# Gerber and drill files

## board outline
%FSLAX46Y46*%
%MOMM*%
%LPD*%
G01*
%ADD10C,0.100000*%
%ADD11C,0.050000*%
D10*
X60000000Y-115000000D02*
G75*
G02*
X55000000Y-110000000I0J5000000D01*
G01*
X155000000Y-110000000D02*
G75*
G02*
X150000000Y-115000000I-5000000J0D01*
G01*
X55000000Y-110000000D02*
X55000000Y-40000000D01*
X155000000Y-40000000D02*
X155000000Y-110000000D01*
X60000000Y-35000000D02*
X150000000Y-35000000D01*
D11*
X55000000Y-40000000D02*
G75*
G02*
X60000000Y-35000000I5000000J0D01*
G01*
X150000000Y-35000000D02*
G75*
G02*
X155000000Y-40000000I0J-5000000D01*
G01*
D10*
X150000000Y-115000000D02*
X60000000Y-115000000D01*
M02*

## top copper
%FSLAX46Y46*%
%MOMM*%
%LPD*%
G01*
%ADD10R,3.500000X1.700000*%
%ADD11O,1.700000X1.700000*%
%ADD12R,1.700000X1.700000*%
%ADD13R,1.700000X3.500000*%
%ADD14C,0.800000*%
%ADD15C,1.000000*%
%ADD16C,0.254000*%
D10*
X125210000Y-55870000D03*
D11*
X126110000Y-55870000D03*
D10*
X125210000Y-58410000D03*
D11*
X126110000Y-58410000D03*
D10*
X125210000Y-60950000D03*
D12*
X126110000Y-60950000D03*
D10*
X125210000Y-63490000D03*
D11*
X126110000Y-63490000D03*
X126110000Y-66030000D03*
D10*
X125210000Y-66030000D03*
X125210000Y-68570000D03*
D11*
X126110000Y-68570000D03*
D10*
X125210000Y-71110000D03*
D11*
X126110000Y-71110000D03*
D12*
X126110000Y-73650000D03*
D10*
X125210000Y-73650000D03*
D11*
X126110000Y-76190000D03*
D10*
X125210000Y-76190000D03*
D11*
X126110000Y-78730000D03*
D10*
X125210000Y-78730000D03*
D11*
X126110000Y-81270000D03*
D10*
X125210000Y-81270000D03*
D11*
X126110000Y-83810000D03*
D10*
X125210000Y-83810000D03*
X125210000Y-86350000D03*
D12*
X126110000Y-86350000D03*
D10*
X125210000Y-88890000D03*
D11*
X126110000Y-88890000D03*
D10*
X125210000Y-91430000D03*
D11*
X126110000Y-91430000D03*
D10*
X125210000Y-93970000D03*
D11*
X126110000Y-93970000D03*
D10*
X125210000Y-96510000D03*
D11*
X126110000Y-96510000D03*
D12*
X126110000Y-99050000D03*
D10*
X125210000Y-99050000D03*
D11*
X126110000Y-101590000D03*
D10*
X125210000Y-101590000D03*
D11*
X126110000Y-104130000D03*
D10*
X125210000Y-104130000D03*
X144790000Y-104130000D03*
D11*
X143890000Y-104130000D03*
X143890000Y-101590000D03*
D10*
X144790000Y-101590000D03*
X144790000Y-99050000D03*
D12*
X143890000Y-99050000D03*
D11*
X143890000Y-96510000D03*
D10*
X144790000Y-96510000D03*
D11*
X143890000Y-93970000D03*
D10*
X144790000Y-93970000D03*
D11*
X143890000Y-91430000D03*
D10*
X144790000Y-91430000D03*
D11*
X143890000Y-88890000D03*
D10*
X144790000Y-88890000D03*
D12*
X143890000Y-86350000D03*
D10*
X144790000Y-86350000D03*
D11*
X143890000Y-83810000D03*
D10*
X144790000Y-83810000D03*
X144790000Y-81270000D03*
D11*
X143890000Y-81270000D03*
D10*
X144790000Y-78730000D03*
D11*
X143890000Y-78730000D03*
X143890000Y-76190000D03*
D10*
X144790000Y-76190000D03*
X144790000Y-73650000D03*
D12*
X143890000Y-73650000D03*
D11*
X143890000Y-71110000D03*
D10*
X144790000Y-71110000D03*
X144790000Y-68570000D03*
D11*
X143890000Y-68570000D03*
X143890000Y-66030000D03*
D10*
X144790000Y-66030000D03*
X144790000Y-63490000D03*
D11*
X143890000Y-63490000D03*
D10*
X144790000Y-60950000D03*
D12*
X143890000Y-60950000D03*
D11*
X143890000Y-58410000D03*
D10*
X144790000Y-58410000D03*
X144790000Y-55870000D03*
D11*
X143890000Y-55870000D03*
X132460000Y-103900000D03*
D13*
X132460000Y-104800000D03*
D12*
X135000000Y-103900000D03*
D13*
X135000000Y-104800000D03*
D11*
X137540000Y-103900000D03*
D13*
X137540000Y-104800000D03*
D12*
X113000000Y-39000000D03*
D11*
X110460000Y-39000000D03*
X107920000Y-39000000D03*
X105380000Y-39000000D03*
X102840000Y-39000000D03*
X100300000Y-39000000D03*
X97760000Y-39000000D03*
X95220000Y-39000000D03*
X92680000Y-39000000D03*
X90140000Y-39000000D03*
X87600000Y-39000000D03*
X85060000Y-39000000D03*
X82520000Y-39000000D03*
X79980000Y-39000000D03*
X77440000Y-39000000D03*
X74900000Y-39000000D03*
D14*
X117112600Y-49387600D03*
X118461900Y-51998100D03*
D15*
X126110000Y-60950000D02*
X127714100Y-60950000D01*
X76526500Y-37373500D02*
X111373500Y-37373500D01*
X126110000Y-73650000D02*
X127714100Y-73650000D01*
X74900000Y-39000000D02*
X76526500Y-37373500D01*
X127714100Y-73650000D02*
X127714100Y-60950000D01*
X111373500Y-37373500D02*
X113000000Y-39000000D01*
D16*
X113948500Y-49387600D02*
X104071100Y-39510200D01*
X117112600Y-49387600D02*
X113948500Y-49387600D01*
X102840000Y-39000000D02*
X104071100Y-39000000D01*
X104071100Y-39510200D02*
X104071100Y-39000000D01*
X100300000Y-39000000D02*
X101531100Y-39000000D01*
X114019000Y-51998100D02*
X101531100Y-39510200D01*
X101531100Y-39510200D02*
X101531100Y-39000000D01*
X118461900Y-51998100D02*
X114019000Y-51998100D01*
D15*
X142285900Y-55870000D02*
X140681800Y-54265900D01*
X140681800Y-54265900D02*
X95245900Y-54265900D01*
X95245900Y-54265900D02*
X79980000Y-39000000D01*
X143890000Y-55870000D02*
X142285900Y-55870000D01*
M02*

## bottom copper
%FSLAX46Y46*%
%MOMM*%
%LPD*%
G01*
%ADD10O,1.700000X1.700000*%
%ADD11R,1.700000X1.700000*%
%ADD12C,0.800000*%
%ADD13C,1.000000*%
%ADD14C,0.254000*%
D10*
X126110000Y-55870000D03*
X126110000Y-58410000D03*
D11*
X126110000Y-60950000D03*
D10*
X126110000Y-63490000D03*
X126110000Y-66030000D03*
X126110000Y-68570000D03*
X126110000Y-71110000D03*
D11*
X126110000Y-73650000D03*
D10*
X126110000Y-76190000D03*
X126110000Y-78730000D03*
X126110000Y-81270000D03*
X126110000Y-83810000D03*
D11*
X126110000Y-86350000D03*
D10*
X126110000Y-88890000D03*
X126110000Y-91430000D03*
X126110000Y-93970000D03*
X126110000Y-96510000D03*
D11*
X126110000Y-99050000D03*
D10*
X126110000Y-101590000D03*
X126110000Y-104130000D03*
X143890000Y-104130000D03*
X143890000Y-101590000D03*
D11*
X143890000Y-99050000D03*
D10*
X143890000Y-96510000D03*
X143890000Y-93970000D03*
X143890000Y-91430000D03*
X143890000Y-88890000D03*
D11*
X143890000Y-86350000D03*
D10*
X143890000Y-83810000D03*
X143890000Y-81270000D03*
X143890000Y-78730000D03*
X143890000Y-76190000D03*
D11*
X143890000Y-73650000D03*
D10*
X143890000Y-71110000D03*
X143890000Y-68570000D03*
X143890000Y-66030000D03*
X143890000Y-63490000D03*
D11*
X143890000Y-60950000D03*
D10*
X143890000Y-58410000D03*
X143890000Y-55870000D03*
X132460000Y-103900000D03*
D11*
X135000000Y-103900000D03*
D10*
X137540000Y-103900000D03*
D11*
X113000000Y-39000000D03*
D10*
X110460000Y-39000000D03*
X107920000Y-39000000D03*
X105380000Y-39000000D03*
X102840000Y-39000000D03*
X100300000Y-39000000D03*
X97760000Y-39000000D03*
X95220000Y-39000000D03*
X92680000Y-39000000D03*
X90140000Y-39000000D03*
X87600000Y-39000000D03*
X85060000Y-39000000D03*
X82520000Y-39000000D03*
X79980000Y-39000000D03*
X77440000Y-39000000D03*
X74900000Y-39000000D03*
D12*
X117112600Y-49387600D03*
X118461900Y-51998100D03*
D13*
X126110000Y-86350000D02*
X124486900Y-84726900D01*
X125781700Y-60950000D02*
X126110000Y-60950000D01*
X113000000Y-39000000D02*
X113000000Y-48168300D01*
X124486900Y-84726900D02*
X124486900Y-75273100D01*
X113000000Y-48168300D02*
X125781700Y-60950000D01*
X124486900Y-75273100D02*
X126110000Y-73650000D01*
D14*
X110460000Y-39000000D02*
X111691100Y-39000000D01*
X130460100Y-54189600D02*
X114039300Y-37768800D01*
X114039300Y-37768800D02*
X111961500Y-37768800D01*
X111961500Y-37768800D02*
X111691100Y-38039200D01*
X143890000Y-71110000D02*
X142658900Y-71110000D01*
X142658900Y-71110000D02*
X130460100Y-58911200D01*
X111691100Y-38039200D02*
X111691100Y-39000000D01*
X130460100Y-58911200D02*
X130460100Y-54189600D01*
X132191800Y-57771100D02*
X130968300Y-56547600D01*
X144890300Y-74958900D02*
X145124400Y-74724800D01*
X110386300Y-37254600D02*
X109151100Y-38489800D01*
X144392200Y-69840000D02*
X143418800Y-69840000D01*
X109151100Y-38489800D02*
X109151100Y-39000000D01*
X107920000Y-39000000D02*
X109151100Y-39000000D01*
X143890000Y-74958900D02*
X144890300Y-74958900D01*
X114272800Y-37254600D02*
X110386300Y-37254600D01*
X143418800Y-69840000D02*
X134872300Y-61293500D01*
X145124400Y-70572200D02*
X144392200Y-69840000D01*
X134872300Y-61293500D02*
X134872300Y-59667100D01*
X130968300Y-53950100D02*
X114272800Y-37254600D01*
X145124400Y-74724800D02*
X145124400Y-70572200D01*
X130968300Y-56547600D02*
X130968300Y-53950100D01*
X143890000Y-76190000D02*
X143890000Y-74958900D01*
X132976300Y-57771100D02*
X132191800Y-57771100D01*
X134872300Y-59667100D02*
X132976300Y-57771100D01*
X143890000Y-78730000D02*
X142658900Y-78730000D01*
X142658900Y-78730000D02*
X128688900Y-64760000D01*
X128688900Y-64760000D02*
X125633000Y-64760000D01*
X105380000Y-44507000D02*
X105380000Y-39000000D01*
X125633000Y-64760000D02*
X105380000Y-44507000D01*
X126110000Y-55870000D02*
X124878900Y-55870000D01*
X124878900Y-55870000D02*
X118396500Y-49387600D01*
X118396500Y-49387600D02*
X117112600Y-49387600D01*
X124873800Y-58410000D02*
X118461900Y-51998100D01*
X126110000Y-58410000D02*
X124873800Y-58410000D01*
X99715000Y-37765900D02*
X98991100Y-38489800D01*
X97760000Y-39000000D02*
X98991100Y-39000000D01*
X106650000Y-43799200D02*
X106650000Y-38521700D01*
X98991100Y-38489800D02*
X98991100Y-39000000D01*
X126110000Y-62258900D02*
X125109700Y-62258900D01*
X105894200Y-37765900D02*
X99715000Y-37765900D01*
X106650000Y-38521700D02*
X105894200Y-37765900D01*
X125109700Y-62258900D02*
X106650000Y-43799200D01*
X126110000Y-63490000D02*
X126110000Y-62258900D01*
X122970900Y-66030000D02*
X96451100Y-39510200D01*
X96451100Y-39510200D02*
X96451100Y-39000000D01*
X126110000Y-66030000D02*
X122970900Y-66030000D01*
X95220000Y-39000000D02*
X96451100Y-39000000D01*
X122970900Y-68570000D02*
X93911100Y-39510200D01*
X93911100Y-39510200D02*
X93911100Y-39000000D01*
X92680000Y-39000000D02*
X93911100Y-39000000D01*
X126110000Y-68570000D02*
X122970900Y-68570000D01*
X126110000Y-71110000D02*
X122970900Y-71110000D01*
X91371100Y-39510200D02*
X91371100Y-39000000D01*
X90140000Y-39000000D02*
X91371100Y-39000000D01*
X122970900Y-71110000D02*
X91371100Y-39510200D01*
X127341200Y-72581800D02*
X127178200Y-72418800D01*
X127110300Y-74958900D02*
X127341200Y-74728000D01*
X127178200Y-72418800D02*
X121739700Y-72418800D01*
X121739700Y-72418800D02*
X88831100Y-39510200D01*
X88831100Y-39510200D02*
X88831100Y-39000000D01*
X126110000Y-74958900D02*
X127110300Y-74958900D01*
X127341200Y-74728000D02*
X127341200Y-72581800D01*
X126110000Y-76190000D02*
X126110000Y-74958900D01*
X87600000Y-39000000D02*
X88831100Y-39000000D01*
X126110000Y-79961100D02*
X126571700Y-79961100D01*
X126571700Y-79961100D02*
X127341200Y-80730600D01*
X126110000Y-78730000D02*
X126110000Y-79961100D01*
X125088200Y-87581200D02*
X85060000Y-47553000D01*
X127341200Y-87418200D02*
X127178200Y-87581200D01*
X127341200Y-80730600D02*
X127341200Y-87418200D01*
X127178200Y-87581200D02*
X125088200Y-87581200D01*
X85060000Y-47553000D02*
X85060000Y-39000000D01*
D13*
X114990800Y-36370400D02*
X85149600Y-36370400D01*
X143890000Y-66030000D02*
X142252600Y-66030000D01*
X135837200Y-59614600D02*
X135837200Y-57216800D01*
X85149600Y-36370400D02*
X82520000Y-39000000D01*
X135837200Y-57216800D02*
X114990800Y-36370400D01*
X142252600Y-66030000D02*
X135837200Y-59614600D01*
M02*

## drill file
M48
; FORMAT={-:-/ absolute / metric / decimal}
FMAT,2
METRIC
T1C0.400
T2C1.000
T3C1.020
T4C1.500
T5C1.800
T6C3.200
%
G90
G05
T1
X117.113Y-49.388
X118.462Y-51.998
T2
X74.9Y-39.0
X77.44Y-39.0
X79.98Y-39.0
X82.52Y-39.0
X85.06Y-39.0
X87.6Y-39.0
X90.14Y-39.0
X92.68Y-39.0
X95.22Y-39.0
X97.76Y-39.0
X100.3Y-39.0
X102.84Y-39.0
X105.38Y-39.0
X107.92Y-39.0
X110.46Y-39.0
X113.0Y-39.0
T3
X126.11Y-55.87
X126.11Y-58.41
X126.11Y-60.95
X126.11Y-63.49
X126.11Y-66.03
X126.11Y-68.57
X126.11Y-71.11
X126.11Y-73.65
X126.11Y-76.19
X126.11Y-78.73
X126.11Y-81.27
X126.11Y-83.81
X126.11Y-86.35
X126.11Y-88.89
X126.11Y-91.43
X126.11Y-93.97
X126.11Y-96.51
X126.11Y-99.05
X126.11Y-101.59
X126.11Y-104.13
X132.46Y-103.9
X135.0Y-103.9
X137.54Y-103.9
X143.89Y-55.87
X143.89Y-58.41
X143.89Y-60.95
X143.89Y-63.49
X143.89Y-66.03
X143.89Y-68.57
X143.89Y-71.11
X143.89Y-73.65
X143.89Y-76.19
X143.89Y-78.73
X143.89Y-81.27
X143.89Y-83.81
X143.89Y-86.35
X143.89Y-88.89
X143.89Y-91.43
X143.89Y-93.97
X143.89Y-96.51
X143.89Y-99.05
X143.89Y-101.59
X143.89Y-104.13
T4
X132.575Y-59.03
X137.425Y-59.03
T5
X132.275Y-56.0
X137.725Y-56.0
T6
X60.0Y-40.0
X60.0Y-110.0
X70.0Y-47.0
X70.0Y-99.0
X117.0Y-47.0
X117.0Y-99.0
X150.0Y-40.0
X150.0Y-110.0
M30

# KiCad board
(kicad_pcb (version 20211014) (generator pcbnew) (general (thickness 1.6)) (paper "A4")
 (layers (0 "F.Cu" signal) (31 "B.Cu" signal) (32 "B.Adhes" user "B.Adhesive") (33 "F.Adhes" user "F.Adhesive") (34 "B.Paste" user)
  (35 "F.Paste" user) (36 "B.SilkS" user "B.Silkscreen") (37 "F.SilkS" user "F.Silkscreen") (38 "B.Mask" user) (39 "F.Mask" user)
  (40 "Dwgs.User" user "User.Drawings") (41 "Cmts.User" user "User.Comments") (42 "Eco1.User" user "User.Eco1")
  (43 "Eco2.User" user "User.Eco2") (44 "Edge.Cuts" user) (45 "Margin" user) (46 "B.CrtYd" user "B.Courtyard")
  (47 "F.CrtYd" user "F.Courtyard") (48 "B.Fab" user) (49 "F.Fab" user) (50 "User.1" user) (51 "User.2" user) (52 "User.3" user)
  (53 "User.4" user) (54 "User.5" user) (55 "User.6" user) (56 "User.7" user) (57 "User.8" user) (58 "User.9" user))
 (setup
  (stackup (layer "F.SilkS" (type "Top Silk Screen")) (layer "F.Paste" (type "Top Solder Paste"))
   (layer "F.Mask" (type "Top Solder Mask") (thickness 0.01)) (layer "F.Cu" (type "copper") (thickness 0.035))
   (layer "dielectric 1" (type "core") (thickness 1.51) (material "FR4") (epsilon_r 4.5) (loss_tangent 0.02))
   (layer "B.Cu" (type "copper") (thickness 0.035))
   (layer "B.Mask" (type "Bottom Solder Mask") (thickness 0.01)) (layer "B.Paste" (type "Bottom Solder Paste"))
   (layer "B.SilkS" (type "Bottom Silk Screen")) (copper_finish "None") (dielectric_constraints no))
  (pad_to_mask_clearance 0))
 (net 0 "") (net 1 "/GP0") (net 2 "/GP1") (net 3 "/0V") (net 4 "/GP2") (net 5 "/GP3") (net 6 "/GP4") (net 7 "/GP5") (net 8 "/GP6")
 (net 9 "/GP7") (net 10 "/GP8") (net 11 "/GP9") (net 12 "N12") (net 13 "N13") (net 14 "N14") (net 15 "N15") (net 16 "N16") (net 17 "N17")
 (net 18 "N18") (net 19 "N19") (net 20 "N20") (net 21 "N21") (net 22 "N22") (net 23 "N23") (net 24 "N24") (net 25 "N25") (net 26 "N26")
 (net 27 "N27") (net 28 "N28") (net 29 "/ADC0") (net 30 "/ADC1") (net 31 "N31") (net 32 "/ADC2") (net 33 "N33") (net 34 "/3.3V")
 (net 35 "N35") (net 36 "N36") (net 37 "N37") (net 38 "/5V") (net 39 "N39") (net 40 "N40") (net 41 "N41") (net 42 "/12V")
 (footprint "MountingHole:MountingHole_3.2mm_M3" (layer "F.Cu") (at 117 99)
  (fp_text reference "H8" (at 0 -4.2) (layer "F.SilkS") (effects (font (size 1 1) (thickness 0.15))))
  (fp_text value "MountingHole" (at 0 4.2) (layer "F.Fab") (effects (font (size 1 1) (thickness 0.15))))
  (pad "" np_thru_hole circle (at 0 0) (size 3.2 3.2) (drill 3.2) (layers *.Cu *.Mask)))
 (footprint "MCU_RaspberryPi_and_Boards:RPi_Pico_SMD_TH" (layer "F.Cu") (at 135 80)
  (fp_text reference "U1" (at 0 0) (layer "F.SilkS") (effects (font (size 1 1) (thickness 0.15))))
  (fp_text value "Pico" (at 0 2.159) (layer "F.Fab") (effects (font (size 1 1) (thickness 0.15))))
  (pad "" np_thru_hole oval (at -2.725 -24) (size 1.8 1.8) (drill 1.8) (layers *.Cu *.Mask))
  (pad "" np_thru_hole oval (at -2.425 -20.97) (size 1.5 1.5) (drill 1.5) (layers *.Cu *.Mask))
  (pad "" np_thru_hole oval (at 2.425 -20.97) (size 1.5 1.5) (drill 1.5) (layers *.Cu *.Mask))
  (pad "" np_thru_hole oval (at 2.725 -24) (size 1.8 1.8) (drill 1.8) (layers *.Cu *.Mask))
  (pad "1" smd rect (at -8.89 -24.13) (size 3.5 1.7) (drill (offset -0.9 0)) (layers "F.Cu" "F.Mask") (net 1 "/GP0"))
  (pad "1" thru_hole oval (at -8.89 -24.13) (size 1.7 1.7) (drill 1.02) (layers *.Cu *.Mask) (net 1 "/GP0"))
  (pad "2" smd rect (at -8.89 -21.59) (size 3.5 1.7) (drill (offset -0.9 0)) (layers "F.Cu" "F.Mask") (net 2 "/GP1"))
  (pad "2" thru_hole oval (at -8.89 -21.59) (size 1.7 1.7) (drill 1.02) (layers *.Cu *.Mask) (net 2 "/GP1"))
  (pad "3" smd rect (at -8.89 -19.05) (size 3.5 1.7) (drill (offset -0.9 0)) (layers "F.Cu" "F.Mask") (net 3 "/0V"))
  (pad "3" thru_hole rect (at -8.89 -19.05) (size 1.7 1.7) (drill 1.02) (layers *.Cu *.Mask) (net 3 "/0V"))
  (pad "4" smd rect (at -8.89 -16.51) (size 3.5 1.7) (drill (offset -0.9 0)) (layers "F.Cu" "F.Mask") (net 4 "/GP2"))
  (pad "4" thru_hole oval (at -8.89 -16.51) (size 1.7 1.7) (drill 1.02) (layers *.Cu *.Mask) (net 4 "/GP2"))
  (pad "5" thru_hole oval (at -8.89 -13.97) (size 1.7 1.7) (drill 1.02) (layers *.Cu *.Mask) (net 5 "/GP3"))
  (pad "5" smd rect (at -8.89 -13.97) (size 3.5 1.7) (drill (offset -0.9 0)) (layers "F.Cu" "F.Mask") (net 5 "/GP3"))
  (pad "6" smd rect (at -8.89 -11.43) (size 3.5 1.7) (drill (offset -0.9 0)) (layers "F.Cu" "F.Mask") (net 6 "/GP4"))
  (pad "6" thru_hole oval (at -8.89 -11.43) (size 1.7 1.7) (drill 1.02) (layers *.Cu *.Mask) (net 6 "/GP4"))
  (pad "7" smd rect (at -8.89 -8.89) (size 3.5 1.7) (drill (offset -0.9 0)) (layers "F.Cu" "F.Mask") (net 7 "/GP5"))
  (pad "7" thru_hole oval (at -8.89 -8.89) (size 1.7 1.7) (drill 1.02) (layers *.Cu *.Mask) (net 7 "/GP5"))
  (pad "8" thru_hole rect (at -8.89 -6.35) (size 1.7 1.7) (drill 1.02) (layers *.Cu *.Mask) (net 3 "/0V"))
  (pad "8" smd rect (at -8.89 -6.35) (size 3.5 1.7) (drill (offset -0.9 0)) (layers "F.Cu" "F.Mask") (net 3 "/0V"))
  (pad "9" thru_hole oval (at -8.89 -3.81) (size 1.7 1.7) (drill 1.02) (layers *.Cu *.Mask) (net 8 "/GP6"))
  (pad "9" smd rect (at -8.89 -3.81) (size 3.5 1.7) (drill (offset -0.9 0)) (layers "F.Cu" "F.Mask") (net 8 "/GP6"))
  (pad "10" thru_hole oval (at -8.89 -1.27) (size 1.7 1.7) (drill 1.02) (layers *.Cu *.Mask) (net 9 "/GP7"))
  (pad "10" smd rect (at -8.89 -1.27) (size 3.5 1.7) (drill (offset -0.9 0)) (layers "F.Cu" "F.Mask") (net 9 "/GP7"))
  (pad "11" thru_hole oval (at -8.89 1.27) (size 1.7 1.7) (drill 1.02) (layers *.Cu *.Mask) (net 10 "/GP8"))
  (pad "11" smd rect (at -8.89 1.27) (size 3.5 1.7) (drill (offset -0.9 0)) (layers "F.Cu" "F.Mask") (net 10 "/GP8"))
  (pad "12" thru_hole oval (at -8.89 3.81) (size 1.7 1.7) (drill 1.02) (layers *.Cu *.Mask) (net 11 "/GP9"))
  (pad "12" smd rect (at -8.89 3.81) (size 3.5 1.7) (drill (offset -0.9 0)) (layers "F.Cu" "F.Mask") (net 11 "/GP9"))
  (pad "13" smd rect (at -8.89 6.35) (size 3.5 1.7) (drill (offset -0.9 0)) (layers "F.Cu" "F.Mask") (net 3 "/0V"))
  (pad "13" thru_hole rect (at -8.89 6.35) (size 1.7 1.7) (drill 1.02) (layers *.Cu *.Mask) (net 3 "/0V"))
  (pad "14" smd rect (at -8.89 8.89) (size 3.5 1.7) (drill (offset -0.9 0)) (layers "F.Cu" "F.Mask") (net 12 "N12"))
  (pad "14" thru_hole oval (at -8.89 8.89) (size 1.7 1.7) (drill 1.02) (layers *.Cu *.Mask) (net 12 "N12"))
  (pad "15" smd rect (at -8.89 11.43) (size 3.5 1.7) (drill (offset -0.9 0)) (layers "F.Cu" "F.Mask") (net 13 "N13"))
  (pad "15" thru_hole oval (at -8.89 11.43) (size 1.7 1.7) (drill 1.02) (layers *.Cu *.Mask) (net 13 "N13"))
  (pad "16" smd rect (at -8.89 13.97) (size 3.5 1.7) (drill (offset -0.9 0)) (layers "F.Cu" "F.Mask") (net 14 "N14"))
  (pad "16" thru_hole oval (at -8.89 13.97) (size 1.7 1.7) (drill 1.02) (layers *.Cu *.Mask) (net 14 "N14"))
  (pad "17" smd rect (at -8.89 16.51) (size 3.5 1.7) (drill (offset -0.9 0)) (layers "F.Cu" "F.Mask") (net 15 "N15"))
  (pad "17" thru_hole oval (at -8.89 16.51) (size 1.7 1.7) (drill 1.02) (layers *.Cu *.Mask) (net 15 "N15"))
  (pad "18" thru_hole rect (at -8.89 19.05) (size 1.7 1.7) (drill 1.02) (layers *.Cu *.Mask) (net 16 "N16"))
  (pad "18" smd rect (at -8.89 19.05) (size 3.5 1.7) (drill (offset -0.9 0)) (layers "F.Cu" "F.Mask") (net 16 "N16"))
  (pad "19" thru_hole oval (at -8.89 21.59) (size 1.7 1.7) (drill 1.02) (layers *.Cu *.Mask) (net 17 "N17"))
  (pad "19" smd rect (at -8.89 21.59) (size 3.5 1.7) (drill (offset -0.9 0)) (layers "F.Cu" "F.Mask") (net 17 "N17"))
  (pad "20" thru_hole oval (at -8.89 24.13) (size 1.7 1.7) (drill 1.02) (layers *.Cu *.Mask) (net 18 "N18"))
  (pad "20" smd rect (at -8.89 24.13) (size 3.5 1.7) (drill (offset -0.9 0)) (layers "F.Cu" "F.Mask") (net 18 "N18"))
  (pad "21" smd rect (at 8.89 24.13) (size 3.5 1.7) (drill (offset 0.9 0)) (layers "F.Cu" "F.Mask") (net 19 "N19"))
  (pad "21" thru_hole oval (at 8.89 24.13) (size 1.7 1.7) (drill 1.02) (layers *.Cu *.Mask) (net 19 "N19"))
  (pad "22" thru_hole oval (at 8.89 21.59) (size 1.7 1.7) (drill 1.02) (layers *.Cu *.Mask) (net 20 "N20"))
  (pad "22" smd rect (at 8.89 21.59) (size 3.5 1.7) (drill (offset 0.9 0)) (layers "F.Cu" "F.Mask") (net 20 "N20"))
  (pad "23" smd rect (at 8.89 19.05) (size 3.5 1.7) (drill (offset 0.9 0)) (layers "F.Cu" "F.Mask") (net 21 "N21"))
  (pad "23" thru_hole rect (at 8.89 19.05) (size 1.7 1.7) (drill 1.02) (layers *.Cu *.Mask) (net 21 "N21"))
  (pad "24" thru_hole oval (at 8.89 16.51) (size 1.7 1.7) (drill 1.02) (layers *.Cu *.Mask) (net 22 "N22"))
  (pad "24" smd rect (at 8.89 16.51) (size 3.5 1.7) (drill (offset 0.9 0)) (layers "F.Cu" "F.Mask") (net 22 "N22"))
  (pad "25" thru_hole oval (at 8.89 13.97) (size 1.7 1.7) (drill 1.02) (layers *.Cu *.Mask) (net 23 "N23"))
  (pad "25" smd rect (at 8.89 13.97) (size 3.5 1.7) (drill (offset 0.9 0)) (layers "F.Cu" "F.Mask") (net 23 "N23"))
  (pad "26" thru_hole oval (at 8.89 11.43) (size 1.7 1.7) (drill 1.02) (layers *.Cu *.Mask) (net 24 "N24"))
  (pad "26" smd rect (at 8.89 11.43) (size 3.5 1.7) (drill (offset 0.9 0)) (layers "F.Cu" "F.Mask") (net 24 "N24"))
  (pad "27" thru_hole oval (at 8.89 8.89) (size 1.7 1.7) (drill 1.02) (layers *.Cu *.Mask) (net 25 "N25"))
  (pad "27" smd rect (at 8.89 8.89) (size 3.5 1.7) (drill (offset 0.9 0)) (layers "F.Cu" "F.Mask") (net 25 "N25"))
  (pad "28" thru_hole rect (at 8.89 6.35) (size 1.7 1.7) (drill 1.02) (layers *.Cu *.Mask) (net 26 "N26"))
  (pad "28" smd rect (at 8.89 6.35) (size 3.5 1.7) (drill (offset 0.9 0)) (layers "F.Cu" "F.Mask") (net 26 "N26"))
  (pad "29" thru_hole oval (at 8.89 3.81) (size 1.7 1.7) (drill 1.02) (layers *.Cu *.Mask) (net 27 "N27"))
  (pad "29" smd rect (at 8.89 3.81) (size 3.5 1.7) (drill (offset 0.9 0)) (layers "F.Cu" "F.Mask") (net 27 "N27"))
  (pad "30" smd rect (at 8.89 1.27) (size 3.5 1.7) (drill (offset 0.9 0)) (layers "F.Cu" "F.Mask") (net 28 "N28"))
  (pad "30" thru_hole oval (at 8.89 1.27) (size 1.7 1.7) (drill 1.02) (layers *.Cu *.Mask) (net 28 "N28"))
  (pad "31" smd rect (at 8.89 -1.27) (size 3.5 1.7) (drill (offset 0.9 0)) (layers "F.Cu" "F.Mask") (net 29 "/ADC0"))
  (pad "31" thru_hole oval (at 8.89 -1.27) (size 1.7 1.7) (drill 1.02) (layers *.Cu *.Mask) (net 29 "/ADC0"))
  (pad "32" thru_hole oval (at 8.89 -3.81) (size 1.7 1.7) (drill 1.02) (layers *.Cu *.Mask) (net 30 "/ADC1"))
  (pad "32" smd rect (at 8.89 -3.81) (size 3.5 1.7) (drill (offset 0.9 0)) (layers "F.Cu" "F.Mask") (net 30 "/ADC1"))
  (pad "33" smd rect (at 8.89 -6.35) (size 3.5 1.7) (drill (offset 0.9 0)) (layers "F.Cu" "F.Mask") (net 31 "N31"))
  (pad "33" thru_hole rect (at 8.89 -6.35) (size 1.7 1.7) (drill 1.02) (layers *.Cu *.Mask) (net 31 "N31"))
  (pad "34" thru_hole oval (at 8.89 -8.89) (size 1.7 1.7) (drill 1.02) (layers *.Cu *.Mask) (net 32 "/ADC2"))
  (pad "34" smd rect (at 8.89 -8.89) (size 3.5 1.7) (drill (offset 0.9 0)) (layers "F.Cu" "F.Mask") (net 32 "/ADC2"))
  (pad "35" smd rect (at 8.89 -11.43) (size 3.5 1.7) (drill (offset 0.9 0)) (layers "F.Cu" "F.Mask") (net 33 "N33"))
  (pad "35" thru_hole oval (at 8.89 -11.43) (size 1.7 1.7) (drill 1.02) (layers *.Cu *.Mask) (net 33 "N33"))
  (pad "36" thru_hole oval (at 8.89 -13.97) (size 1.7 1.7) (drill 1.02) (layers *.Cu *.Mask) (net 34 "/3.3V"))
  (pad "36" smd rect (at 8.89 -13.97) (size 3.5 1.7) (drill (offset 0.9 0)) (layers "F.Cu" "F.Mask") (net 34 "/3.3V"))
  (pad "37" smd rect (at 8.89 -16.51) (size 3.5 1.7) (drill (offset 0.9 0)) (layers "F.Cu" "F.Mask") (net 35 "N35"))
  (pad "37" thru_hole oval (at 8.89 -16.51) (size 1.7 1.7) (drill 1.02) (layers *.Cu *.Mask) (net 35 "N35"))
  (pad "38" smd rect (at 8.89 -19.05) (size 3.5 1.7) (drill (offset 0.9 0)) (layers "F.Cu" "F.Mask") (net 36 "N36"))
  (pad "38" thru_hole rect (at 8.89 -19.05) (size 1.7 1.7) (drill 1.02) (layers *.Cu *.Mask) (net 36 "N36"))
  (pad "39" thru_hole oval (at 8.89 -21.59) (size 1.7 1.7) (drill 1.02) (layers *.Cu *.Mask) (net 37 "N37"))
  (pad "39" smd rect (at 8.89 -21.59) (size 3.5 1.7) (drill (offset 0.9 0)) (layers "F.Cu" "F.Mask") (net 37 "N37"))
  (pad "40" smd rect (at 8.89 -24.13) (size 3.5 1.7) (drill (offset 0.9 0)) (layers "F.Cu" "F.Mask") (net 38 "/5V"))
  (pad "40" thru_hole oval (at 8.89 -24.13) (size 1.7 1.7) (drill 1.02) (layers *.Cu *.Mask) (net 38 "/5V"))
  (pad "41" thru_hole oval (at -2.54 23.9) (size 1.7 1.7) (drill 1.02) (layers *.Cu *.Mask) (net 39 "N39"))
  (pad "41" smd rect (at -2.54 23.9 90) (size 3.5 1.7) (drill (offset -0.9 0)) (layers "F.Cu" "F.Mask") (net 39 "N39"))
  (pad "42" thru_hole rect (at 0 23.9) (size 1.7 1.7) (drill 1.02) (layers *.Cu *.Mask) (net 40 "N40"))
  (pad "42" smd rect (at 0 23.9 90) (size 3.5 1.7) (drill (offset -0.9 0)) (layers "F.Cu" "F.Mask") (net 40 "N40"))
  (pad "43" thru_hole oval (at 2.54 23.9) (size 1.7 1.7) (drill 1.02) (layers *.Cu *.Mask) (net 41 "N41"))
  (pad "43" smd rect (at 2.54 23.9 90) (size 3.5 1.7) (drill (offset -0.9 0)) (layers "F.Cu" "F.Mask") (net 41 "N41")))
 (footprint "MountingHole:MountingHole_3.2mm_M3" (layer "F.Cu") (at 70 99)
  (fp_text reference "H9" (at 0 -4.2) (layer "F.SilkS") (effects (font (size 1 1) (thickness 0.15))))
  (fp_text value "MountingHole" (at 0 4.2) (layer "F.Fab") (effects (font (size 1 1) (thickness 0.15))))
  (pad "" np_thru_hole circle (at 0 0) (size 3.2 3.2) (drill 3.2) (layers *.Cu *.Mask)))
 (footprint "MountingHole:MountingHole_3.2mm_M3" (layer "F.Cu") (at 117 47)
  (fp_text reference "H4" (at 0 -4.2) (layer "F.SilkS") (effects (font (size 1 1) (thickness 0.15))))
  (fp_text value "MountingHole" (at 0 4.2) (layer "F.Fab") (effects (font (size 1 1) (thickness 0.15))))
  (pad "" np_thru_hole circle (at 0 0) (size 3.2 3.2) (drill 3.2) (layers *.Cu *.Mask)))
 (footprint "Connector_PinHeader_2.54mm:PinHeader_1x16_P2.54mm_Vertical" (layer "F.Cu") (at 113 39 -90)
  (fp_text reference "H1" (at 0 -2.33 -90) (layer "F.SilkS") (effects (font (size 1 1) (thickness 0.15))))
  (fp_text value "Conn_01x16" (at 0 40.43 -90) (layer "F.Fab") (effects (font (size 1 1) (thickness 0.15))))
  (pad "1" thru_hole rect (at 0 0 270) (size 1.7 1.7) (drill 1) (layers *.Cu *.Mask) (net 3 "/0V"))
  (pad "2" thru_hole oval (at 0 2.54 270) (size 1.7 1.7) (drill 1) (layers *.Cu *.Mask) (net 32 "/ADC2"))
  (pad "3" thru_hole oval (at 0 5.08 270) (size 1.7 1.7) (drill 1) (layers *.Cu *.Mask) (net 30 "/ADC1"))
  (pad "4" thru_hole oval (at 0 7.62 270) (size 1.7 1.7) (drill 1) (layers *.Cu *.Mask) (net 29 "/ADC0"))
  (pad "5" thru_hole oval (at 0 10.16 270) (size 1.7 1.7) (drill 1) (layers *.Cu *.Mask) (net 1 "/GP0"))
  (pad "6" thru_hole oval (at 0 12.7 270) (size 1.7 1.7) (drill 1) (layers *.Cu *.Mask) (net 2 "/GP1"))
  (pad "7" thru_hole oval (at 0 15.24 270) (size 1.7 1.7) (drill 1) (layers *.Cu *.Mask) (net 4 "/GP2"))
  (pad "8" thru_hole oval (at 0 17.78 270) (size 1.7 1.7) (drill 1) (layers *.Cu *.Mask) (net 5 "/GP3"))
  (pad "9" thru_hole oval (at 0 20.32 270) (size 1.7 1.7) (drill 1) (layers *.Cu *.Mask) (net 6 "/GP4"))
  (pad "10" thru_hole oval (at 0 22.86 270) (size 1.7 1.7) (drill 1) (layers *.Cu *.Mask) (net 7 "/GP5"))
  (pad "11" thru_hole oval (at 0 25.4 270) (size 1.7 1.7) (drill 1) (layers *.Cu *.Mask) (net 8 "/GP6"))
  (pad "12" thru_hole oval (at 0 27.94 270) (size 1.7 1.7) (drill 1) (layers *.Cu *.Mask) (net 9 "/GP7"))
  (pad "13" thru_hole oval (at 0 30.48 270) (size 1.7 1.7) (drill 1) (layers *.Cu *.Mask) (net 34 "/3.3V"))
  (pad "14" thru_hole oval (at 0 33.02 270) (size 1.7 1.7) (drill 1) (layers *.Cu *.Mask) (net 38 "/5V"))
  (pad "15" thru_hole oval (at 0 35.56 270) (size 1.7 1.7) (drill 1) (layers *.Cu *.Mask) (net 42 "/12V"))
  (pad "16" thru_hole oval (at 0 38.1 270) (size 1.7 1.7) (drill 1) (layers *.Cu *.Mask) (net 3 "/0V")))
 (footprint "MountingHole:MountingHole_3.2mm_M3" (layer "F.Cu") (at 60 40)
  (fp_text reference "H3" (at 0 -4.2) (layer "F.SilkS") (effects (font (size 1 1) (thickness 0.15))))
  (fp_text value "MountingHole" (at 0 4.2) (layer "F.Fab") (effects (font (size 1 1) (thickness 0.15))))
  (pad "" np_thru_hole circle (at 0 0) (size 3.2 3.2) (drill 3.2) (layers *.Cu *.Mask)))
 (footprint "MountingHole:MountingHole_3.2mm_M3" (layer "F.Cu") (at 70 47)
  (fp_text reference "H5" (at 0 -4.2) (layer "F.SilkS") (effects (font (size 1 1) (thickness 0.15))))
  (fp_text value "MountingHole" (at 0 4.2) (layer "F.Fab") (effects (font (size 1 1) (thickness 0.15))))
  (pad "" np_thru_hole circle (at 0 0) (size 3.2 3.2) (drill 3.2) (layers *.Cu *.Mask)))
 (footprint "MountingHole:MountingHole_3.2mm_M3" (layer "F.Cu") (at 150 110)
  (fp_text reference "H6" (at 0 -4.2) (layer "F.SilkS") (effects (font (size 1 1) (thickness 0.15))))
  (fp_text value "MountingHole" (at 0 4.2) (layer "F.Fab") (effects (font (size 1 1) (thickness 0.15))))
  (pad "" np_thru_hole circle (at 0 0) (size 3.2 3.2) (drill 3.2) (layers *.Cu *.Mask)))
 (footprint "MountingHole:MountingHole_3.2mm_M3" (layer "F.Cu") (at 60 110)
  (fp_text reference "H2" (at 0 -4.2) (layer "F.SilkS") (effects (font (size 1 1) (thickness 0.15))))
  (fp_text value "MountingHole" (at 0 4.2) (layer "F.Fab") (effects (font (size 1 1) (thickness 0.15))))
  (pad "" np_thru_hole circle (at 0 0) (size 3.2 3.2) (drill 3.2) (layers *.Cu *.Mask)))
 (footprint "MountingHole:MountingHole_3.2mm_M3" (layer "F.Cu") (at 150 40)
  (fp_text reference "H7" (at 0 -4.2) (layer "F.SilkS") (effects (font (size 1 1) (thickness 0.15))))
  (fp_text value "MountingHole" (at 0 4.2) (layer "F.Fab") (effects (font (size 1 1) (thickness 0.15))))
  (pad "" np_thru_hole circle (at 0 0) (size 3.2 3.2) (drill 3.2) (layers *.Cu *.Mask)))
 (gr_arc (start 60 115) (mid 56.464466 113.535534) (end 55 110) (layer "Edge.Cuts") (width 0.1))
 (gr_arc (start 155 110) (mid 153.535534 113.535534) (end 150 115) (layer "Edge.Cuts") (width 0.1))
 (gr_line (start 55 110) (end 55 40) (layer "Edge.Cuts") (width 0.1))
 (gr_line (start 155 40) (end 155 110) (layer "Edge.Cuts") (width 0.1))
 (gr_line (start 60 35) (end 150 35) (layer "Edge.Cuts") (width 0.1))
 (gr_arc (start 55 40) (mid 56.464466 36.464466) (end 60 35) (layer "Edge.Cuts") (width 0.05))
 (gr_arc (start 150 35) (mid 153.535534 36.464466) (end 155 40) (layer "Edge.Cuts") (width 0.05))
 (gr_line (start 150 115) (end 60 115) (layer "Edge.Cuts") (width 0.1))
 (segment (start 126.11 60.95) (end 127.7141 60.95) (width 1) (layer "F.Cu") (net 3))
 (segment (start 76.5265 37.3735) (end 111.3735 37.3735) (width 1) (layer "F.Cu") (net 3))
 (segment (start 126.11 73.65) (end 127.7141 73.65) (width 1) (layer "F.Cu") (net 3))
 (segment (start 74.9 39) (end 76.5265 37.3735) (width 1) (layer "F.Cu") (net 3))
 (segment (start 127.7141 73.65) (end 127.7141 60.95) (width 1) (layer "F.Cu") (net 3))
 (segment (start 111.3735 37.3735) (end 113 39) (width 1) (layer "F.Cu") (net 3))
 (segment (start 126.11 86.35) (end 124.4869 84.7269) (width 1) (layer "B.Cu") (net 3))
 (segment (start 125.7817 60.95) (end 126.11 60.95) (width 1) (layer "B.Cu") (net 3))
 (segment (start 113 39) (end 113 48.1683) (width 1) (layer "B.Cu") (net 3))
 (segment (start 124.4869 84.7269) (end 124.4869 75.2731) (width 1) (layer "B.Cu") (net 3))
 (segment (start 113 48.1683) (end 125.7817 60.95) (width 1) (layer "B.Cu") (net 3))
 (segment (start 124.4869 75.2731) (end 126.11 73.65) (width 1) (layer "B.Cu") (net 3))
 (segment (start 110.46 39) (end 111.6911 39) (width 0.254) (layer "B.Cu") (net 32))
 (segment (start 130.4601 54.1896) (end 114.0393 37.7688) (width 0.254) (layer "B.Cu") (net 32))
 (segment (start 114.0393 37.7688) (end 111.9615 37.7688) (width 0.254) (layer "B.Cu") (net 32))
 (segment (start 111.9615 37.7688) (end 111.6911 38.0392) (width 0.254) (layer "B.Cu") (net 32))
 (segment (start 143.89 71.11) (end 142.6589 71.11) (width 0.254) (layer "B.Cu") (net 32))
 (segment (start 142.6589 71.11) (end 130.4601 58.9112) (width 0.254) (layer "B.Cu") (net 32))
 (segment (start 111.6911 38.0392) (end 111.6911 39) (width 0.254) (layer "B.Cu") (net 32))
 (segment (start 130.4601 58.9112) (end 130.4601 54.1896) (width 0.254) (layer "B.Cu") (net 32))
 (segment (start 132.1918 57.7711) (end 130.9683 56.5476) (width 0.254) (layer "B.Cu") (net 30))
 (segment (start 144.8903 74.9589) (end 145.1244 74.7248) (width 0.254) (layer "B.Cu") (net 30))
 (segment (start 110.3863 37.2546) (end 109.1511 38.4898) (width 0.254) (layer "B.Cu") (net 30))
 (segment (start 144.3922 69.84) (end 143.4188 69.84) (width 0.254) (layer "B.Cu") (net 30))
 (segment (start 109.1511 38.4898) (end 109.1511 39) (width 0.254) (layer "B.Cu") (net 30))
 (segment (start 107.92 39) (end 109.1511 39) (width 0.254) (layer "B.Cu") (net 30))
 (segment (start 143.89 74.9589) (end 144.8903 74.9589) (width 0.254) (layer "B.Cu") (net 30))
 (segment (start 114.2728 37.2546) (end 110.3863 37.2546) (width 0.254) (layer "B.Cu") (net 30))
 (segment (start 143.4188 69.84) (end 134.8723 61.2935) (width 0.254) (layer "B.Cu") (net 30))
 (segment (start 145.1244 70.5722) (end 144.3922 69.84) (width 0.254) (layer "B.Cu") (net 30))
 (segment (start 134.8723 61.2935) (end 134.8723 59.6671) (width 0.254) (layer "B.Cu") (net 30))
 (segment (start 130.9683 53.9501) (end 114.2728 37.2546) (width 0.254) (layer "B.Cu") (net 30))
 (segment (start 145.1244 74.7248) (end 145.1244 70.5722) (width 0.254) (layer "B.Cu") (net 30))
 (segment (start 130.9683 56.5476) (end 130.9683 53.9501) (width 0.254) (layer "B.Cu") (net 30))
 (segment (start 143.89 76.19) (end 143.89 74.9589) (width 0.254) (layer "B.Cu") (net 30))
 (segment (start 132.9763 57.7711) (end 132.1918 57.7711) (width 0.254) (layer "B.Cu") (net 30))
 (segment (start 134.8723 59.6671) (end 132.9763 57.7711) (width 0.254) (layer "B.Cu") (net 30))
 (segment (start 143.89 78.73) (end 142.6589 78.73) (width 0.254) (layer "B.Cu") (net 29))
 (segment (start 142.6589 78.73) (end 128.6889 64.76) (width 0.254) (layer "B.Cu") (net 29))
 (segment (start 128.6889 64.76) (end 125.633 64.76) (width 0.254) (layer "B.Cu") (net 29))
 (segment (start 105.38 44.507) (end 105.38 39) (width 0.254) (layer "B.Cu") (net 29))
 (segment (start 125.633 64.76) (end 105.38 44.507) (width 0.254) (layer "B.Cu") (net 29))
 (segment (start 113.9485 49.3876) (end 104.0711 39.5102) (width 0.254) (layer "F.Cu") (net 1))
 (segment (start 117.1126 49.3876) (end 113.9485 49.3876) (width 0.254) (layer "F.Cu") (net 1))
 (segment (start 102.84 39) (end 104.0711 39) (width 0.254) (layer "F.Cu") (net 1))
 (segment (start 104.0711 39.5102) (end 104.0711 39) (width 0.254) (layer "F.Cu") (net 1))
 (via (at 117.1126 49.3876) (size 0.8) (drill 0.4) (layers "F.Cu" "B.Cu") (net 1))
 (segment (start 126.11 55.87) (end 124.8789 55.87) (width 0.254) (layer "B.Cu") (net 1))
 (segment (start 124.8789 55.87) (end 118.3965 49.3876) (width 0.254) (layer "B.Cu") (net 1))
 (segment (start 118.3965 49.3876) (end 117.1126 49.3876) (width 0.254) (layer "B.Cu") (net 1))
 (segment (start 100.3 39) (end 101.5311 39) (width 0.254) (layer "F.Cu") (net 2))
 (segment (start 114.019 51.9981) (end 101.5311 39.5102) (width 0.254) (layer "F.Cu") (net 2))
 (segment (start 101.5311 39.5102) (end 101.5311 39) (width 0.254) (layer "F.Cu") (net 2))
 (segment (start 118.4619 51.9981) (end 114.019 51.9981) (width 0.254) (layer "F.Cu") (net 2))
 (via (at 118.4619 51.9981) (size 0.8) (drill 0.4) (layers "F.Cu" "B.Cu") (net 2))
 (segment (start 124.8738 58.41) (end 118.4619 51.9981) (width 0.254) (layer "B.Cu") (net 2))
 (segment (start 126.11 58.41) (end 124.8738 58.41) (width 0.254) (layer "B.Cu") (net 2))
 (segment (start 99.715 37.7659) (end 98.9911 38.4898) (width 0.254) (layer "B.Cu") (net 4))
 (segment (start 97.76 39) (end 98.9911 39) (width 0.254) (layer "B.Cu") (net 4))
 (segment (start 106.65 43.7992) (end 106.65 38.5217) (width 0.254) (layer "B.Cu") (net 4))
 (segment (start 98.9911 38.4898) (end 98.9911 39) (width 0.254) (layer "B.Cu") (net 4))
 (segment (start 126.11 62.2589) (end 125.1097 62.2589) (width 0.254) (layer "B.Cu") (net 4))
 (segment (start 105.8942 37.7659) (end 99.715 37.7659) (width 0.254) (layer "B.Cu") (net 4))
 (segment (start 106.65 38.5217) (end 105.8942 37.7659) (width 0.254) (layer "B.Cu") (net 4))
 (segment (start 125.1097 62.2589) (end 106.65 43.7992) (width 0.254) (layer "B.Cu") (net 4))
 (segment (start 126.11 63.49) (end 126.11 62.2589) (width 0.254) (layer "B.Cu") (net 4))
 (segment (start 122.9709 66.03) (end 96.4511 39.5102) (width 0.254) (layer "B.Cu") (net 5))
 (segment (start 96.4511 39.5102) (end 96.4511 39) (width 0.254) (layer "B.Cu") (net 5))
 (segment (start 126.11 66.03) (end 122.9709 66.03) (width 0.254) (layer "B.Cu") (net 5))
 (segment (start 95.22 39) (end 96.4511 39) (width 0.254) (layer "B.Cu") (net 5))
 (segment (start 122.9709 68.57) (end 93.9111 39.5102) (width 0.254) (layer "B.Cu") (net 6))
 (segment (start 93.9111 39.5102) (end 93.9111 39) (width 0.254) (layer "B.Cu") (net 6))
 (segment (start 92.68 39) (end 93.9111 39) (width 0.254) (layer "B.Cu") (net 6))
 (segment (start 126.11 68.57) (end 122.9709 68.57) (width 0.254) (layer "B.Cu") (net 6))
 (segment (start 126.11 71.11) (end 122.9709 71.11) (width 0.254) (layer "B.Cu") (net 7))
 (segment (start 91.3711 39.5102) (end 91.3711 39) (width 0.254) (layer "B.Cu") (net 7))
 (segment (start 90.14 39) (end 91.3711 39) (width 0.254) (layer "B.Cu") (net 7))
 (segment (start 122.9709 71.11) (end 91.3711 39.5102) (width 0.254) (layer "B.Cu") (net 7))
 (segment (start 127.3412 72.5818) (end 127.1782 72.4188) (width 0.254) (layer "B.Cu") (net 8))
 (segment (start 127.1103 74.9589) (end 127.3412 74.728) (width 0.254) (layer "B.Cu") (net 8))
 (segment (start 127.1782 72.4188) (end 121.7397 72.4188) (width 0.254) (layer "B.Cu") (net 8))
 (segment (start 121.7397 72.4188) (end 88.8311 39.5102) (width 0.254) (layer "B.Cu") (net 8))
 (segment (start 88.8311 39.5102) (end 88.8311 39) (width 0.254) (layer "B.Cu") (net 8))
 (segment (start 126.11 74.9589) (end 127.1103 74.9589) (width 0.254) (layer "B.Cu") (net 8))
 (segment (start 127.3412 74.728) (end 127.3412 72.5818) (width 0.254) (layer "B.Cu") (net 8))
 (segment (start 126.11 76.19) (end 126.11 74.9589) (width 0.254) (layer "B.Cu") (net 8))
 (segment (start 87.6 39) (end 88.8311 39) (width 0.254) (layer "B.Cu") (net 8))
 (segment (start 126.11 79.9611) (end 126.5717 79.9611) (width 0.254) (layer "B.Cu") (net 9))
 (segment (start 126.5717 79.9611) (end 127.3412 80.7306) (width 0.254) (layer "B.Cu") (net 9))
 (segment (start 126.11 78.73) (end 126.11 79.9611) (width 0.254) (layer "B.Cu") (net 9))
 (segment (start 125.0882 87.5812) (end 85.06 47.553) (width 0.254) (layer "B.Cu") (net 9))
 (segment (start 127.3412 87.4182) (end 127.1782 87.5812) (width 0.254) (layer "B.Cu") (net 9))
 (segment (start 127.3412 80.7306) (end 127.3412 87.4182) (width 0.254) (layer "B.Cu") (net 9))
 (segment (start 127.1782 87.5812) (end 125.0882 87.5812) (width 0.254) (layer "B.Cu") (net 9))
 (segment (start 85.06 47.553) (end 85.06 39) (width 0.254) (layer "B.Cu") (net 9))
 (segment (start 114.9908 36.3704) (end 85.1496 36.3704) (width 1) (layer "B.Cu") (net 34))
 (segment (start 143.89 66.03) (end 142.2526 66.03) (width 1) (layer "B.Cu") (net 34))
 (segment (start 135.8372 59.6146) (end 135.8372 57.2168) (width 1) (layer "B.Cu") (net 34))
 (segment (start 85.1496 36.3704) (end 82.52 39) (width 1) (layer "B.Cu") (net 34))
 (segment (start 135.8372 57.2168) (end 114.9908 36.3704) (width 1) (layer "B.Cu") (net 34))
 (segment (start 142.2526 66.03) (end 135.8372 59.6146) (width 1) (layer "B.Cu") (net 34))
 (segment (start 142.2859 55.87) (end 140.6818 54.2659) (width 1) (layer "F.Cu") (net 38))
 (segment (start 140.6818 54.2659) (end 95.2459 54.2659) (width 1) (layer "F.Cu") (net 38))
 (segment (start 95.2459 54.2659) (end 79.98 39) (width 1) (layer "F.Cu") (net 38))
 (segment (start 143.89 55.87) (end 142.2859 55.87) (width 1) (layer "F.Cu") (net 38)))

